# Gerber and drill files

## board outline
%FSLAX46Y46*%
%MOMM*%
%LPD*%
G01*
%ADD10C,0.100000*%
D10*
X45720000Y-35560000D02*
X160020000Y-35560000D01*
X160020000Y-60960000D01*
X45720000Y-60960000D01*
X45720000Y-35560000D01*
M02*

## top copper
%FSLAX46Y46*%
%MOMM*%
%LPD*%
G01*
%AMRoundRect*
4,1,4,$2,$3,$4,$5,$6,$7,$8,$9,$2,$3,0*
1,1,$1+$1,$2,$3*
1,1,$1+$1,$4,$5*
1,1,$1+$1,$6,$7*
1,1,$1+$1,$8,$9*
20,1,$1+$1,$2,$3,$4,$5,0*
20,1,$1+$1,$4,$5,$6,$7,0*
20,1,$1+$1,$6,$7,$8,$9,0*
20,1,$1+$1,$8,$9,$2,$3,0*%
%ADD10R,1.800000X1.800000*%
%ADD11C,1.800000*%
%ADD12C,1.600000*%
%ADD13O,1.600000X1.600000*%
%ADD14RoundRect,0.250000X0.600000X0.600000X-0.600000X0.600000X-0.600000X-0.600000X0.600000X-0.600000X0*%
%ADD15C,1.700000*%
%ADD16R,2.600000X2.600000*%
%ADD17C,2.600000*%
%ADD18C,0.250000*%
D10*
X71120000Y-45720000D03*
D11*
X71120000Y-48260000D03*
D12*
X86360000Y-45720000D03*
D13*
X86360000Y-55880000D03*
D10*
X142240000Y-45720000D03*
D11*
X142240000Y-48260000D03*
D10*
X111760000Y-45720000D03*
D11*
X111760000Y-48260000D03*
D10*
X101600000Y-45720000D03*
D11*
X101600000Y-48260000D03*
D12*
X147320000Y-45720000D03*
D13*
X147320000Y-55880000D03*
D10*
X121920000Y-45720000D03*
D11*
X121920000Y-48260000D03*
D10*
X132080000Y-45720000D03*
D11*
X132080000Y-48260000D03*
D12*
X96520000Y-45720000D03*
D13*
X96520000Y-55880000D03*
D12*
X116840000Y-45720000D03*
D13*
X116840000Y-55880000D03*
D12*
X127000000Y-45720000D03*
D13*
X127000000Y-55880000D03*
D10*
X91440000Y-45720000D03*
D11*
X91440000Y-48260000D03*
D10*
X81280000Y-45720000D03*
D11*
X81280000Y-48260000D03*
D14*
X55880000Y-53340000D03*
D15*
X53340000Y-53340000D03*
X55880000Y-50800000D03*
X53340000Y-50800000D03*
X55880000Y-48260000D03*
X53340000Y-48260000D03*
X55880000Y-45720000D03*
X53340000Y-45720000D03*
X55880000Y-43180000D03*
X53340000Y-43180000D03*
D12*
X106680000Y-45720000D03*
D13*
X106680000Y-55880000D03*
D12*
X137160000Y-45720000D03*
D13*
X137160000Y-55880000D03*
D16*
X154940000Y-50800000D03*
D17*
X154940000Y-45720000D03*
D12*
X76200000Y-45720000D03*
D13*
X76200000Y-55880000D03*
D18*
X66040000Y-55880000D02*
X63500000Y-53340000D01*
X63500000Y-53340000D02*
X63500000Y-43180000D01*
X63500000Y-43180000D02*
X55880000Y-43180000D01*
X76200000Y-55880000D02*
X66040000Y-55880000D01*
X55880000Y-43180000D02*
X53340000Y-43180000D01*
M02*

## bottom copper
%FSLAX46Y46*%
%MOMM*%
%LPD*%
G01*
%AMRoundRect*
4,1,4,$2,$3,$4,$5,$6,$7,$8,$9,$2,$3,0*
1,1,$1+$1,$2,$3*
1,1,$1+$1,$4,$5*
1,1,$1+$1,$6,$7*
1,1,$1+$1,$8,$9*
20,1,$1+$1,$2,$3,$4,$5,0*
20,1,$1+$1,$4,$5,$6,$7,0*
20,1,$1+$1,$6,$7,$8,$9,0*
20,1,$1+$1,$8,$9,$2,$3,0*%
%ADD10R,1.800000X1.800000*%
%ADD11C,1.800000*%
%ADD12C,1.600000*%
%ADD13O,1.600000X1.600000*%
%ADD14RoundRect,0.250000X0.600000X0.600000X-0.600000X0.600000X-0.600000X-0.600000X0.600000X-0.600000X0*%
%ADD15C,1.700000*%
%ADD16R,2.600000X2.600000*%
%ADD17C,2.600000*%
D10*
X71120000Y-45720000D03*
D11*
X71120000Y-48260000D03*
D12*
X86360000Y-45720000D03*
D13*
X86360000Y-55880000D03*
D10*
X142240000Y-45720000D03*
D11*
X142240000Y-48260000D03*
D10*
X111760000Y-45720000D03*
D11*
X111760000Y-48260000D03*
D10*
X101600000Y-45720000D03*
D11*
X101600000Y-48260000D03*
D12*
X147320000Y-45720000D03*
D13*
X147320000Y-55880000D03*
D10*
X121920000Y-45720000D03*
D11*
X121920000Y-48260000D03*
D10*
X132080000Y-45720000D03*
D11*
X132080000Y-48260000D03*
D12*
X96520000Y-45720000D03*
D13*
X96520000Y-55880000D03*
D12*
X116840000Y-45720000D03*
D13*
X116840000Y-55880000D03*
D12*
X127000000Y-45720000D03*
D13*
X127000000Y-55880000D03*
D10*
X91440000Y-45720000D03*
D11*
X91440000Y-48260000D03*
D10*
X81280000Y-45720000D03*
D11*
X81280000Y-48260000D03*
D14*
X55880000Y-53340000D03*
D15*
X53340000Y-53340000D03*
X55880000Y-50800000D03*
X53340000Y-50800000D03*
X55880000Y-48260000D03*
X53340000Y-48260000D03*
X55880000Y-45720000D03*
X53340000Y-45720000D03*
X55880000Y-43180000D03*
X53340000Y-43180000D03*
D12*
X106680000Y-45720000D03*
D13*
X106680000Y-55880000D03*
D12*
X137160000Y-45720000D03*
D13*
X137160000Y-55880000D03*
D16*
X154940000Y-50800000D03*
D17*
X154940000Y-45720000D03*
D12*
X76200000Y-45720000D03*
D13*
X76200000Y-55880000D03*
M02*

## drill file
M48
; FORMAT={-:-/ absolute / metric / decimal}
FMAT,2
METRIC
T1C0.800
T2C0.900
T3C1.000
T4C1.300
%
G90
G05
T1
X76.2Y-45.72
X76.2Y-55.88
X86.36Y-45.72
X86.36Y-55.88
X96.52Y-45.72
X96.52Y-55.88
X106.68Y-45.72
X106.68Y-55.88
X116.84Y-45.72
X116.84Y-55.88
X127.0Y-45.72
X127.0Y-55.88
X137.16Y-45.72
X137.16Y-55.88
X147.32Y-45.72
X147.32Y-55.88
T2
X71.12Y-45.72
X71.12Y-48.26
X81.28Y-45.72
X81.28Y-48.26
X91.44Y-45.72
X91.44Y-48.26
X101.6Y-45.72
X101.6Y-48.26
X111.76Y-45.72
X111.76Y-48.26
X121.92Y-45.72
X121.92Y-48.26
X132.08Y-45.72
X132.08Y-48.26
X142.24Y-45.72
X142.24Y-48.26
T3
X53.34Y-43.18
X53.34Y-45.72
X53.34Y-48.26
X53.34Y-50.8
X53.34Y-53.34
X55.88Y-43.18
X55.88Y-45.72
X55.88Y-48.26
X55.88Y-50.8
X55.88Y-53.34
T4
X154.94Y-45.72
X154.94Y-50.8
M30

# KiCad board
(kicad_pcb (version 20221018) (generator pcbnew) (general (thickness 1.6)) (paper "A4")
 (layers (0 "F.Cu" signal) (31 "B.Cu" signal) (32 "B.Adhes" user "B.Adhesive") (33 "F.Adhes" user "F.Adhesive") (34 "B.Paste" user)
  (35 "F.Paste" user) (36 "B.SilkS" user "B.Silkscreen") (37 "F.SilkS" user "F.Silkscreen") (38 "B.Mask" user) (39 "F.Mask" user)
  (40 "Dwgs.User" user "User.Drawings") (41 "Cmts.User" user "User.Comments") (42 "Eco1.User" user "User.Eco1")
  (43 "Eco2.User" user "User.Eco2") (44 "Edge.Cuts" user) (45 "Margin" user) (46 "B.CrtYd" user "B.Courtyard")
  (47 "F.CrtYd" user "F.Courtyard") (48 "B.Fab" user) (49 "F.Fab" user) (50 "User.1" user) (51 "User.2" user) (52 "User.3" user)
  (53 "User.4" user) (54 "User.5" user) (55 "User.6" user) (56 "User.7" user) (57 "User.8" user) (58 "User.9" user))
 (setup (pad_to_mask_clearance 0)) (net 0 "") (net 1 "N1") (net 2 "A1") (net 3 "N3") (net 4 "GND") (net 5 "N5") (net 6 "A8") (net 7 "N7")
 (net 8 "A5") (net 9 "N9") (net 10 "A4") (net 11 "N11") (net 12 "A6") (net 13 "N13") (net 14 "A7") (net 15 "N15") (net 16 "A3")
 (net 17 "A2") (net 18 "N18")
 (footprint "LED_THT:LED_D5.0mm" (layer "F.Cu") (at 71.12 45.72 -90)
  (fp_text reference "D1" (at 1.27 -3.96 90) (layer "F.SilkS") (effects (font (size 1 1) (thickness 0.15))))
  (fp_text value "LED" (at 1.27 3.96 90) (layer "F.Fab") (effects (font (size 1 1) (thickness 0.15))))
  (pad "1" thru_hole rect (at 0 0 270) (size 1.8 1.8) (drill 0.9) (layers "*.Cu" "*.Mask") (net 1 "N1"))
  (pad "2" thru_hole circle (at 2.54 0 270) (size 1.8 1.8) (drill 0.9) (layers "*.Cu" "*.Mask") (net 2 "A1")))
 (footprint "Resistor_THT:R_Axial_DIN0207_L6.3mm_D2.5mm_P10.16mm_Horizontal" (layer "F.Cu") (at 86.36 45.72 -90)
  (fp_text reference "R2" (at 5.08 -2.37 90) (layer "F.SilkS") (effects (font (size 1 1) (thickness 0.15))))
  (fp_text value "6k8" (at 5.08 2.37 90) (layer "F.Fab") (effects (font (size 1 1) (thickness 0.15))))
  (pad "1" thru_hole circle (at 0 0 270) (size 1.6 1.6) (drill 0.8) (layers "*.Cu" "*.Mask") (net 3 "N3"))
  (pad "2" thru_hole oval (at 10.16 0 270) (size 1.6 1.6) (drill 0.8) (layers "*.Cu" "*.Mask") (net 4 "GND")))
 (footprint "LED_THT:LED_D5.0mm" (layer "F.Cu") (at 142.24 45.72 -90)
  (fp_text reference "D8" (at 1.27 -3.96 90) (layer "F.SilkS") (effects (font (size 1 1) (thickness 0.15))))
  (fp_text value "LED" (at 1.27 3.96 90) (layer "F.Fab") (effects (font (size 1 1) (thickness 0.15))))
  (pad "1" thru_hole rect (at 0 0 270) (size 1.8 1.8) (drill 0.9) (layers "*.Cu" "*.Mask") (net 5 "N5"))
  (pad "2" thru_hole circle (at 2.54 0 270) (size 1.8 1.8) (drill 0.9) (layers "*.Cu" "*.Mask") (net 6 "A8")))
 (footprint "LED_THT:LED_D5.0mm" (layer "F.Cu") (at 111.76 45.72 -90)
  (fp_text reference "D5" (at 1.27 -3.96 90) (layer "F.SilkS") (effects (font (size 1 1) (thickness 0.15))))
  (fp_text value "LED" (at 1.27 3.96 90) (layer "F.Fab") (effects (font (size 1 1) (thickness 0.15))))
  (pad "1" thru_hole rect (at 0 0 270) (size 1.8 1.8) (drill 0.9) (layers "*.Cu" "*.Mask") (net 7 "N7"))
  (pad "2" thru_hole circle (at 2.54 0 270) (size 1.8 1.8) (drill 0.9) (layers "*.Cu" "*.Mask") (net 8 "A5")))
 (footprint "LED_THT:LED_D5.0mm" (layer "F.Cu") (at 101.6 45.72 -90)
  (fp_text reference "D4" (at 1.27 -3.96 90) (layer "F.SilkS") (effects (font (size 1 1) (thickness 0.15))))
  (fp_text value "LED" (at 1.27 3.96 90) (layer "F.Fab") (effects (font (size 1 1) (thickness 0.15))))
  (pad "1" thru_hole rect (at 0 0 270) (size 1.8 1.8) (drill 0.9) (layers "*.Cu" "*.Mask") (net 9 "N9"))
  (pad "2" thru_hole circle (at 2.54 0 270) (size 1.8 1.8) (drill 0.9) (layers "*.Cu" "*.Mask") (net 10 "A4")))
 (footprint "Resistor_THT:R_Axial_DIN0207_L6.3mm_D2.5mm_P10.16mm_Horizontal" (layer "F.Cu") (at 147.32 45.72 -90)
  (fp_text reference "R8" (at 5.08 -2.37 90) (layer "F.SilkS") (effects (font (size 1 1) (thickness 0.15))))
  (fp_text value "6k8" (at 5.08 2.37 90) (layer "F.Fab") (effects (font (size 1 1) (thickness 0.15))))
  (pad "1" thru_hole circle (at 0 0 270) (size 1.6 1.6) (drill 0.8) (layers "*.Cu" "*.Mask") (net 5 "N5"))
  (pad "2" thru_hole oval (at 10.16 0 270) (size 1.6 1.6) (drill 0.8) (layers "*.Cu" "*.Mask") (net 4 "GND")))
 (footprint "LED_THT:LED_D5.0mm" (layer "F.Cu") (at 121.92 45.72 -90)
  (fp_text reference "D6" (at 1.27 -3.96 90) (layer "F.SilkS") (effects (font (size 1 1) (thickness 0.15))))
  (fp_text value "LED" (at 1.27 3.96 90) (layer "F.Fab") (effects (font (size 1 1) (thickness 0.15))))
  (pad "1" thru_hole rect (at 0 0 270) (size 1.8 1.8) (drill 0.9) (layers "*.Cu" "*.Mask") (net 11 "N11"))
  (pad "2" thru_hole circle (at 2.54 0 270) (size 1.8 1.8) (drill 0.9) (layers "*.Cu" "*.Mask") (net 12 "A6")))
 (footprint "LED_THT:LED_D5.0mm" (layer "F.Cu") (at 132.08 45.72 -90)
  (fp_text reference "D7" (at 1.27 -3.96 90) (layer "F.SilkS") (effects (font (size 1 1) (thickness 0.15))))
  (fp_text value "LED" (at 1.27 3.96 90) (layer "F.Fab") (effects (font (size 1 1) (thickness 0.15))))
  (pad "1" thru_hole rect (at 0 0 270) (size 1.8 1.8) (drill 0.9) (layers "*.Cu" "*.Mask") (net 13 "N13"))
  (pad "2" thru_hole circle (at 2.54 0 270) (size 1.8 1.8) (drill 0.9) (layers "*.Cu" "*.Mask") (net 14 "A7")))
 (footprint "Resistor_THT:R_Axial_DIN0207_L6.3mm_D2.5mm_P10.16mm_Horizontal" (layer "F.Cu") (at 96.52 45.72 -90)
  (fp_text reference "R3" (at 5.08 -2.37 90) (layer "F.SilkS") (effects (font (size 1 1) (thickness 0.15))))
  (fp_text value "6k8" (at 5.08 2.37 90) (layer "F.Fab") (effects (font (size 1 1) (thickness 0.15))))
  (pad "1" thru_hole circle (at 0 0 270) (size 1.6 1.6) (drill 0.8) (layers "*.Cu" "*.Mask") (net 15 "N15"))
  (pad "2" thru_hole oval (at 10.16 0 270) (size 1.6 1.6) (drill 0.8) (layers "*.Cu" "*.Mask") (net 4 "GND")))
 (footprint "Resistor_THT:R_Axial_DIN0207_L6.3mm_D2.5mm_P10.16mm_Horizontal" (layer "F.Cu") (at 116.84 45.72 -90)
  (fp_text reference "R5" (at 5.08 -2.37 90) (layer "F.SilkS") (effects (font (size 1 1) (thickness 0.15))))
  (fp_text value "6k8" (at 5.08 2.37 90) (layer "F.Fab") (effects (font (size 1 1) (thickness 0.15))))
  (pad "1" thru_hole circle (at 0 0 270) (size 1.6 1.6) (drill 0.8) (layers "*.Cu" "*.Mask") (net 7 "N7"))
  (pad "2" thru_hole oval (at 10.16 0 270) (size 1.6 1.6) (drill 0.8) (layers "*.Cu" "*.Mask") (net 4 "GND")))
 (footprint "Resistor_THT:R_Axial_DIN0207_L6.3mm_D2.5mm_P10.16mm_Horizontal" (layer "F.Cu") (at 127 45.72 -90)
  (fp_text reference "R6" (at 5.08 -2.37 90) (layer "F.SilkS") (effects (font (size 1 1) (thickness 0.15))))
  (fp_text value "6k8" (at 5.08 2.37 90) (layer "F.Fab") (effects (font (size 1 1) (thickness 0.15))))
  (pad "1" thru_hole circle (at 0 0 270) (size 1.6 1.6) (drill 0.8) (layers "*.Cu" "*.Mask") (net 11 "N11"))
  (pad "2" thru_hole oval (at 10.16 0 270) (size 1.6 1.6) (drill 0.8) (layers "*.Cu" "*.Mask") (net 4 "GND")))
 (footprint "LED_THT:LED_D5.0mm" (layer "F.Cu") (at 91.44 45.72 -90)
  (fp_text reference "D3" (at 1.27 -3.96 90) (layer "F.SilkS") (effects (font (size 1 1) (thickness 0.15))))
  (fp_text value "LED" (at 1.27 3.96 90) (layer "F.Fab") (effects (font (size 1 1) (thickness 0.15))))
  (pad "1" thru_hole rect (at 0 0 270) (size 1.8 1.8) (drill 0.9) (layers "*.Cu" "*.Mask") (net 15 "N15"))
  (pad "2" thru_hole circle (at 2.54 0 270) (size 1.8 1.8) (drill 0.9) (layers "*.Cu" "*.Mask") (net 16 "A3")))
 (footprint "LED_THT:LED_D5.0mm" (layer "F.Cu") (at 81.28 45.72 -90)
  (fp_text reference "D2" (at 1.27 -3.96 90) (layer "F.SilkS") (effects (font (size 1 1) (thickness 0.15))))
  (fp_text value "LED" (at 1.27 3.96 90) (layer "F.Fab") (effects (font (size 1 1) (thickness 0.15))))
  (pad "1" thru_hole rect (at 0 0 270) (size 1.8 1.8) (drill 0.9) (layers "*.Cu" "*.Mask") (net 3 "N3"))
  (pad "2" thru_hole circle (at 2.54 0 270) (size 1.8 1.8) (drill 0.9) (layers "*.Cu" "*.Mask") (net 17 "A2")))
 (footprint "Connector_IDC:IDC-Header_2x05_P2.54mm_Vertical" (layer "F.Cu") (at 55.88 53.34 180)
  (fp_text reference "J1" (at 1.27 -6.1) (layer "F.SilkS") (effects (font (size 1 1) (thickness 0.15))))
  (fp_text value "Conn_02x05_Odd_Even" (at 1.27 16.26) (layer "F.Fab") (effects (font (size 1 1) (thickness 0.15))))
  (pad "1" thru_hole roundrect (at 0 0 180) (size 1.7 1.7) (drill 1) (layers "*.Cu" "*.Mask") (roundrect_rratio 0.147059) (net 2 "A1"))
  (pad "2" thru_hole circle (at 2.54 0 180) (size 1.7 1.7) (drill 1) (layers "*.Cu" "*.Mask") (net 17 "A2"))
  (pad "3" thru_hole circle (at 0 2.54 180) (size 1.7 1.7) (drill 1) (layers "*.Cu" "*.Mask") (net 16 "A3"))
  (pad "4" thru_hole circle (at 2.54 2.54 180) (size 1.7 1.7) (drill 1) (layers "*.Cu" "*.Mask") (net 10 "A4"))
  (pad "5" thru_hole circle (at 0 5.08 180) (size 1.7 1.7) (drill 1) (layers "*.Cu" "*.Mask") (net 8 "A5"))
  (pad "6" thru_hole circle (at 2.54 5.08 180) (size 1.7 1.7) (drill 1) (layers "*.Cu" "*.Mask") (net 12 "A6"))
  (pad "7" thru_hole circle (at 0 7.62 180) (size 1.7 1.7) (drill 1) (layers "*.Cu" "*.Mask") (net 14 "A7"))
  (pad "8" thru_hole circle (at 2.54 7.62 180) (size 1.7 1.7) (drill 1) (layers "*.Cu" "*.Mask") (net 6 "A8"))
  (pad "9" thru_hole circle (at 0 10.16 180) (size 1.7 1.7) (drill 1) (layers "*.Cu" "*.Mask") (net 4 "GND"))
  (pad "10" thru_hole circle (at 2.54 10.16 180) (size 1.7 1.7) (drill 1) (layers "*.Cu" "*.Mask") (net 4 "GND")))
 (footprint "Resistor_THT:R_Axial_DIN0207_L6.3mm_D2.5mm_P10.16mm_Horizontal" (layer "F.Cu") (at 106.68 45.72 -90)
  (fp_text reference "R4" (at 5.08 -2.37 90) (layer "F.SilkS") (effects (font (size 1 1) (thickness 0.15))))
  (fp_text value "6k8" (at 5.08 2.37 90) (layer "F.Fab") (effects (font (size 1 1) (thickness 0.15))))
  (pad "1" thru_hole circle (at 0 0 270) (size 1.6 1.6) (drill 0.8) (layers "*.Cu" "*.Mask") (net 9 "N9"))
  (pad "2" thru_hole oval (at 10.16 0 270) (size 1.6 1.6) (drill 0.8) (layers "*.Cu" "*.Mask") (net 4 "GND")))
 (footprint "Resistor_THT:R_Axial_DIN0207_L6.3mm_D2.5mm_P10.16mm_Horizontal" (layer "F.Cu") (at 137.16 45.72 -90)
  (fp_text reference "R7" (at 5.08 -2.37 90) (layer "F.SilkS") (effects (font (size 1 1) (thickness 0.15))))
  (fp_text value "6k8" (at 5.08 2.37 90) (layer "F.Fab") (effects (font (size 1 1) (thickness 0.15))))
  (pad "1" thru_hole circle (at 0 0 270) (size 1.6 1.6) (drill 0.8) (layers "*.Cu" "*.Mask") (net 13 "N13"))
  (pad "2" thru_hole oval (at 10.16 0 270) (size 1.6 1.6) (drill 0.8) (layers "*.Cu" "*.Mask") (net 4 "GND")))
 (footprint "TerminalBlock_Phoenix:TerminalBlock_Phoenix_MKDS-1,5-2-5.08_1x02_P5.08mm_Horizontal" (layer "F.Cu") (at 154.94 50.8 90)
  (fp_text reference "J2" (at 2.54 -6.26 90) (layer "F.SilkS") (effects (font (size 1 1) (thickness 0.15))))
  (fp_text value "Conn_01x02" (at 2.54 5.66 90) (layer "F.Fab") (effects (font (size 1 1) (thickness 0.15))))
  (pad "1" thru_hole rect (at 0 0 90) (size 2.6 2.6) (drill 1.3) (layers "*.Cu" "*.Mask") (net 4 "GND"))
  (pad "2" thru_hole circle (at 5.08 0 90) (size 2.6 2.6) (drill 1.3) (layers "*.Cu" "*.Mask") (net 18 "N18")))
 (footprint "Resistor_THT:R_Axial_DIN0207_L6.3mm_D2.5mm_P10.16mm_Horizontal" (layer "F.Cu") (at 76.2 45.72 -90)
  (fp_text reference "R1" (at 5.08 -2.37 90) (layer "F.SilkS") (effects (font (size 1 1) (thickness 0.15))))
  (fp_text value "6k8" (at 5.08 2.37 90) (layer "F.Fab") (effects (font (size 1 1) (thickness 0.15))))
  (pad "1" thru_hole circle (at 0 0 270) (size 1.6 1.6) (drill 0.8) (layers "*.Cu" "*.Mask") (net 1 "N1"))
  (pad "2" thru_hole oval (at 10.16 0 270) (size 1.6 1.6) (drill 0.8) (layers "*.Cu" "*.Mask") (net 4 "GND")))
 (gr_rect (start 45.72 35.56) (end 160.02 60.96) (stroke (width 0.1) (type default)) (fill none) (layer "Edge.Cuts"))
 (segment (start 66.04 55.88) (end 63.5 53.34) (width 0.25) (layer "F.Cu") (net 4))
 (segment (start 63.5 53.34) (end 63.5 43.18) (width 0.25) (layer "F.Cu") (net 4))
 (segment (start 63.5 43.18) (end 55.88 43.18) (width 0.25) (layer "F.Cu") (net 4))
 (segment (start 76.2 55.88) (end 66.04 55.88) (width 0.25) (layer "F.Cu") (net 4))
 (segment (start 55.88 43.18) (end 53.34 43.18) (width 0.25) (layer "F.Cu") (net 4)))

